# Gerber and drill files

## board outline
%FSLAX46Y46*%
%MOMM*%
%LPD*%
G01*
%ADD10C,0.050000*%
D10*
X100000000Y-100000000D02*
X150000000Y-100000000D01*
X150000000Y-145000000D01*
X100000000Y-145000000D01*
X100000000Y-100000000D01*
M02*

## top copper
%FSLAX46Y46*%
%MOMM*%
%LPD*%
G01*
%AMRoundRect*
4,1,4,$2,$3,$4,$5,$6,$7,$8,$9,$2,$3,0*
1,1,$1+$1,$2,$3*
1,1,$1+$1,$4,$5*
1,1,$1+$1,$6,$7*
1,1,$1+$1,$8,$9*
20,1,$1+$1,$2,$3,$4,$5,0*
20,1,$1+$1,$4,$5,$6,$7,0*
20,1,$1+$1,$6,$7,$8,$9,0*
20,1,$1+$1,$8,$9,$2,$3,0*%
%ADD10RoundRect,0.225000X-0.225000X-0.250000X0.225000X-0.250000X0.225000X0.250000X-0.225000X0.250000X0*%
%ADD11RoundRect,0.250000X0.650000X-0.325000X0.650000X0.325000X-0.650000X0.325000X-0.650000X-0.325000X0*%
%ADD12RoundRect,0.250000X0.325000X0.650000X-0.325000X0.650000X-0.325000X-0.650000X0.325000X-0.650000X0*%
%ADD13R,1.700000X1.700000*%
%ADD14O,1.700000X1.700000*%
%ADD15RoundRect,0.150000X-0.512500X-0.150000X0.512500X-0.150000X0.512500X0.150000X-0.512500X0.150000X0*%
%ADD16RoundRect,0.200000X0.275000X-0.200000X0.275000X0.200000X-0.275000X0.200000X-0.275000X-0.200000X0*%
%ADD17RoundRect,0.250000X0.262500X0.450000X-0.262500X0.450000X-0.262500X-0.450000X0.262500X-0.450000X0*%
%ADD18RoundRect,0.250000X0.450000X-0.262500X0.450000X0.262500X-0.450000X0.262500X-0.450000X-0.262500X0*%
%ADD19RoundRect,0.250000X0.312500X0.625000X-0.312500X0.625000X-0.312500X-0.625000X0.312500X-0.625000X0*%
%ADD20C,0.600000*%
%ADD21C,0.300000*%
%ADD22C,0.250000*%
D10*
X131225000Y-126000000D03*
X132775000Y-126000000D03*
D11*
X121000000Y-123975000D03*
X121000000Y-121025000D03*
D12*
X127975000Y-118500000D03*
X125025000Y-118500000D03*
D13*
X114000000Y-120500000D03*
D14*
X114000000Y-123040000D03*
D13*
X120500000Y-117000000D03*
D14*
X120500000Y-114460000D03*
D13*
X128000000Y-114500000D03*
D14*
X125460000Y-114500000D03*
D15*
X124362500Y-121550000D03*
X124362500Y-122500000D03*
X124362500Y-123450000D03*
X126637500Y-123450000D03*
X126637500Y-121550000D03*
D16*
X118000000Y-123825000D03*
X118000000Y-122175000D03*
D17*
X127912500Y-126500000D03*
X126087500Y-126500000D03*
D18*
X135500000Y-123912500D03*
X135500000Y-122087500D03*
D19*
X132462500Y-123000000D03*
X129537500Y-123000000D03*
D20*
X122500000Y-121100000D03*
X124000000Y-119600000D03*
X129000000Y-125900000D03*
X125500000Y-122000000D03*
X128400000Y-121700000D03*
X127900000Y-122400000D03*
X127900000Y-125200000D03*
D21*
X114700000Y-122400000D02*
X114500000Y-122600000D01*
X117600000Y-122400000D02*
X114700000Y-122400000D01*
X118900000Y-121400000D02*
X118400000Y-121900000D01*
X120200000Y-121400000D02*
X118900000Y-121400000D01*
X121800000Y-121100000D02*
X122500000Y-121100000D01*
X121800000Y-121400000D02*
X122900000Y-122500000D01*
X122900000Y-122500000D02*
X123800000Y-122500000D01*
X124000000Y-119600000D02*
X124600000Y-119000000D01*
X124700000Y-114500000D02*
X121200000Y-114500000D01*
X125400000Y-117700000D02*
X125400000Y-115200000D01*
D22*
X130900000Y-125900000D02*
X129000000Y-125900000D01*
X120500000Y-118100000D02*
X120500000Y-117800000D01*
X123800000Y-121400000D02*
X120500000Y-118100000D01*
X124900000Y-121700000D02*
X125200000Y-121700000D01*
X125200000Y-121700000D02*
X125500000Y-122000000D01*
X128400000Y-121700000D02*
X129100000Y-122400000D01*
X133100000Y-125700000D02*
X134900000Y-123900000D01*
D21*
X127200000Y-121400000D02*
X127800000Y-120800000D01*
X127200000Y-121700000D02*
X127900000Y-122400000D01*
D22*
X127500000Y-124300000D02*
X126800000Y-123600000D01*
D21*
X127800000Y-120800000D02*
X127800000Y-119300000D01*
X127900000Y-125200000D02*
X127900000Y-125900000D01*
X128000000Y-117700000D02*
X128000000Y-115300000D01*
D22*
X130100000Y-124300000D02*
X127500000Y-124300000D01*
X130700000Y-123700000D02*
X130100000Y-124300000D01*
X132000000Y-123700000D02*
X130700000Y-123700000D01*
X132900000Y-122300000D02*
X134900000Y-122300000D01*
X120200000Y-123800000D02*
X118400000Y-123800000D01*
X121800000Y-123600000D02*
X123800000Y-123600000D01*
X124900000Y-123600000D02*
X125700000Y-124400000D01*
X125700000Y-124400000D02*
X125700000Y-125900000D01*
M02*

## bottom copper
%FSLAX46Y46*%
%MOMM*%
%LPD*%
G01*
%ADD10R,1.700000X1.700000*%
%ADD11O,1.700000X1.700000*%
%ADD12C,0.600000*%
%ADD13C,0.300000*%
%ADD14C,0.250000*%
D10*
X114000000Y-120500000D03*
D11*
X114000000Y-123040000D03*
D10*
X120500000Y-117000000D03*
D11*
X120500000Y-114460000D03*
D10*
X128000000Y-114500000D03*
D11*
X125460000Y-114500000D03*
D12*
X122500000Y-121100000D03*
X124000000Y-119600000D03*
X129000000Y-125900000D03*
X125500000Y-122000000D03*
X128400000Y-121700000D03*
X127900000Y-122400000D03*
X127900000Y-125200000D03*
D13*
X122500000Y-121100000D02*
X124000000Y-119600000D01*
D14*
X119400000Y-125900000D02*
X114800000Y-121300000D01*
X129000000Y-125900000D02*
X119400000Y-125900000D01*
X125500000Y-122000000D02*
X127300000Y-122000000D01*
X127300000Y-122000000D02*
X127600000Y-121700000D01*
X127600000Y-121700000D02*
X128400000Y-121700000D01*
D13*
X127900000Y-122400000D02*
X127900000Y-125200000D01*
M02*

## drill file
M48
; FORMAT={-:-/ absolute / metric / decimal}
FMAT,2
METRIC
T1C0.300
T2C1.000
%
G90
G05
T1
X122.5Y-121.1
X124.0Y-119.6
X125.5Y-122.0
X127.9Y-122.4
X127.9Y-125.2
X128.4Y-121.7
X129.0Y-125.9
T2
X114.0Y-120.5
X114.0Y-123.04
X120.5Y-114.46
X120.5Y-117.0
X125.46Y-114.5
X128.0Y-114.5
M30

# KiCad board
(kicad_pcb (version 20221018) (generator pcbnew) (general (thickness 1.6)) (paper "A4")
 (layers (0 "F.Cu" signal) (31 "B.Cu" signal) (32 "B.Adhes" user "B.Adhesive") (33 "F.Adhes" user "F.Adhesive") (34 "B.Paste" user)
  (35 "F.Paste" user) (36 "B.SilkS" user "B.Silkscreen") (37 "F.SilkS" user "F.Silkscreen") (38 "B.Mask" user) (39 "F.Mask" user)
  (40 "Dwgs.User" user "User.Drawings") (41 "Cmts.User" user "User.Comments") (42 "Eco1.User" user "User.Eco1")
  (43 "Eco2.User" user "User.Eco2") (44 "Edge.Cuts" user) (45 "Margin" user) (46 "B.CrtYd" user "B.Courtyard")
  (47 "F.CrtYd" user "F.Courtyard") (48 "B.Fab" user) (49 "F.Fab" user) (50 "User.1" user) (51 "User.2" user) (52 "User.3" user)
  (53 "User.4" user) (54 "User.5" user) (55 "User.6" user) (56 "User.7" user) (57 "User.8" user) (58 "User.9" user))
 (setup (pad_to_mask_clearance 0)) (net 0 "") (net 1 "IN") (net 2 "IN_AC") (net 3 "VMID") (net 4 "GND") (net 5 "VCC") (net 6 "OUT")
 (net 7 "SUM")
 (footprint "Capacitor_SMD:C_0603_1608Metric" (layer "F.Cu") (at 132 126)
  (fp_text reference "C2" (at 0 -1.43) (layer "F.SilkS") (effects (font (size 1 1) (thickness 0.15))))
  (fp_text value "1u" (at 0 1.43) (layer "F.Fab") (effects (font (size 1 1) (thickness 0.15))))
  (pad "1" smd roundrect (at -0.775 0) (size 0.9 0.95) (layers "F.Cu" "F.Paste" "F.Mask") (roundrect_rratio 0.25) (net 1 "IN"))
  (pad "2" smd roundrect (at 0.775 0) (size 0.9 0.95) (layers "F.Cu" "F.Paste" "F.Mask") (roundrect_rratio 0.25) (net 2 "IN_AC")))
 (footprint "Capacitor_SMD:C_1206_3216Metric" (layer "F.Cu") (at 121 122.5 90)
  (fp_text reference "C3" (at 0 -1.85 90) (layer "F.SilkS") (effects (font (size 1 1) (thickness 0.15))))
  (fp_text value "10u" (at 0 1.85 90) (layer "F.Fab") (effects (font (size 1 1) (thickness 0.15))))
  (pad "1" smd roundrect (at -1.475 0 90) (size 1.15 1.8) (layers "F.Cu" "F.Paste" "F.Mask") (roundrect_rratio 0.217391) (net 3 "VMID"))
  (pad "2" smd roundrect (at 1.475 0 90) (size 1.15 1.8) (layers "F.Cu" "F.Paste" "F.Mask") (roundrect_rratio 0.217391) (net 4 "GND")))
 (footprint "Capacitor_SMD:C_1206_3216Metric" (layer "F.Cu") (at 126.5 118.5 180)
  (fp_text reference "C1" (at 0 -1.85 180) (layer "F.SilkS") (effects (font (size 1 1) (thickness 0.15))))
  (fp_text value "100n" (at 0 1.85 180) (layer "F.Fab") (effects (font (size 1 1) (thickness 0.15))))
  (pad "1" smd roundrect (at -1.475 0 180) (size 1.15 1.8) (layers "F.Cu" "F.Paste" "F.Mask") (roundrect_rratio 0.217391) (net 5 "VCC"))
  (pad "2" smd roundrect (at 1.475 0 180) (size 1.15 1.8) (layers "F.Cu" "F.Paste" "F.Mask") (roundrect_rratio 0.217391) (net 4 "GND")))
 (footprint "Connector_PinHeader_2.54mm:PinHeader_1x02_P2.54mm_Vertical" (layer "F.Cu") (at 114 120.5)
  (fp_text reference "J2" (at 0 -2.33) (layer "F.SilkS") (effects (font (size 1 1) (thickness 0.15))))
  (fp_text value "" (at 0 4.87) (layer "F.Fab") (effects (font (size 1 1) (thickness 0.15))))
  (pad "1" thru_hole rect (at 0 0) (size 1.7 1.7) (drill 1) (layers "*.Cu" "*.Mask") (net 1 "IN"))
  (pad "2" thru_hole oval (at 0 2.54) (size 1.7 1.7) (drill 1) (layers "*.Cu" "*.Mask") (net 4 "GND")))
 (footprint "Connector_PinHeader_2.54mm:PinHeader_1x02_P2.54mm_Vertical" (layer "F.Cu") (at 120.5 117 180)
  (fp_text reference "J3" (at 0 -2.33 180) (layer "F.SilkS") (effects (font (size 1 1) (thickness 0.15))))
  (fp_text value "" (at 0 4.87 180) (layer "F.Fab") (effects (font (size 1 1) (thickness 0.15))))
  (pad "1" thru_hole rect (at 0 0 180) (size 1.7 1.7) (drill 1) (layers "*.Cu" "*.Mask") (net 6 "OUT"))
  (pad "2" thru_hole oval (at 0 2.54 180) (size 1.7 1.7) (drill 1) (layers "*.Cu" "*.Mask") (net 4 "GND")))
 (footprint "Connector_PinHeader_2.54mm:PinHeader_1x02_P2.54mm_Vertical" (layer "F.Cu") (at 128 114.5 -90)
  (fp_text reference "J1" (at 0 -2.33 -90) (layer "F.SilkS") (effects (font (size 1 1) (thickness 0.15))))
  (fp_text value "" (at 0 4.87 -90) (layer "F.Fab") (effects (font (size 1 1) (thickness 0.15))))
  (pad "1" thru_hole rect (at 0 0 270) (size 1.7 1.7) (drill 1) (layers "*.Cu" "*.Mask") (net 5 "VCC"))
  (pad "2" thru_hole oval (at 0 2.54 270) (size 1.7 1.7) (drill 1) (layers "*.Cu" "*.Mask") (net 4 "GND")))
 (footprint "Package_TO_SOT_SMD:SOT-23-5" (layer "F.Cu") (at 125.5 122.5)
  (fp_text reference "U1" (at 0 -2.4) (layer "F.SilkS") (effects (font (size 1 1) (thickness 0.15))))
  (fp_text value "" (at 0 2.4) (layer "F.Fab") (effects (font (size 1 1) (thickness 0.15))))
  (pad "1" smd roundrect (at -1.1375 -0.95) (size 1.325 0.6) (layers "F.Cu" "F.Paste" "F.Mask") (roundrect_rratio 0.25) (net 6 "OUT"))
  (pad "2" smd roundrect (at -1.1375 0) (size 1.325 0.6) (layers "F.Cu" "F.Paste" "F.Mask") (roundrect_rratio 0.25) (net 4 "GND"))
  (pad "3" smd roundrect (at -1.1375 0.95) (size 1.325 0.6) (layers "F.Cu" "F.Paste" "F.Mask") (roundrect_rratio 0.25) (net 3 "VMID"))
  (pad "4" smd roundrect (at 1.1375 0.95) (size 1.325 0.6) (layers "F.Cu" "F.Paste" "F.Mask") (roundrect_rratio 0.25) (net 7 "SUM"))
  (pad "5" smd roundrect (at 1.1375 -0.95) (size 1.325 0.6) (layers "F.Cu" "F.Paste" "F.Mask") (roundrect_rratio 0.25) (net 5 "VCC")))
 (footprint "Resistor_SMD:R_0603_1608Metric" (layer "F.Cu") (at 118 123 90)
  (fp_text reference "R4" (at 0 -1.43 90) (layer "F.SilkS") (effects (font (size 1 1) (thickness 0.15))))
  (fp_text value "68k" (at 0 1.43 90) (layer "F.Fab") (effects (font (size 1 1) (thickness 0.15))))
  (pad "1" smd roundrect (at -0.825 0 90) (size 0.8 0.95) (layers "F.Cu" "F.Paste" "F.Mask") (roundrect_rratio 0.25) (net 3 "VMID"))
  (pad "2" smd roundrect (at 0.825 0 90) (size 0.8 0.95) (layers "F.Cu" "F.Paste" "F.Mask") (roundrect_rratio 0.25) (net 4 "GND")))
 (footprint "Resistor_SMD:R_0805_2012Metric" (layer "F.Cu") (at 127 126.5 180)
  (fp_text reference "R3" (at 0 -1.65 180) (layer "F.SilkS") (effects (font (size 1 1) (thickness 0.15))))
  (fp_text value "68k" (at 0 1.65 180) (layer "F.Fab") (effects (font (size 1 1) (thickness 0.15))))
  (pad "1" smd roundrect (at -0.9125 0 180) (size 1.025 1.4) (layers "F.Cu" "F.Paste" "F.Mask") (roundrect_rratio 0.243902) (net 5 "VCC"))
  (pad "2" smd roundrect (at 0.9125 0 180) (size 1.025 1.4) (layers "F.Cu" "F.Paste" "F.Mask") (roundrect_rratio 0.243902) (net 3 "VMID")))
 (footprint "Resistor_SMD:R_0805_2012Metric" (layer "F.Cu") (at 135.5 123 90)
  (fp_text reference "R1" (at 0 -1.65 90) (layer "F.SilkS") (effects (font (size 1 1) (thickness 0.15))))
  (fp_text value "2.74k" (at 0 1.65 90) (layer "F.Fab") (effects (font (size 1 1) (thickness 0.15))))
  (pad "1" smd roundrect (at -0.9125 0 90) (size 1.025 1.4) (layers "F.Cu" "F.Paste" "F.Mask") (roundrect_rratio 0.243902) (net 2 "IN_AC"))
  (pad "2" smd roundrect (at 0.9125 0 90) (size 1.025 1.4) (layers "F.Cu" "F.Paste" "F.Mask") (roundrect_rratio 0.243902) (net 7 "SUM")))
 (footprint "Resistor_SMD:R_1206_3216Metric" (layer "F.Cu") (at 131 123 180)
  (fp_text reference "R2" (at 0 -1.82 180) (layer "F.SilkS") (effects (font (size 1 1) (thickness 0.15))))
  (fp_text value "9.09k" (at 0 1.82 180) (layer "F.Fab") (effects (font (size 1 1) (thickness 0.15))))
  (pad "1" smd roundrect (at -1.4625 0 180) (size 1.125 1.75) (layers "F.Cu" "F.Paste" "F.Mask") (roundrect_rratio 0.222222) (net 7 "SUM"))
  (pad "2" smd roundrect (at 1.4625 0 180) (size 1.125 1.75) (layers "F.Cu" "F.Paste" "F.Mask") (roundrect_rratio 0.222222) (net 6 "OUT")))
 (gr_rect (start 100 100) (end 150 145) (stroke (width 0.05) (type default)) (fill none) (layer "Edge.Cuts"))
 (segment (start 114.7 122.4) (end 114.5 122.6) (width 0.3) (layer "F.Cu") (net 4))
 (segment (start 117.6 122.4) (end 114.7 122.4) (width 0.3) (layer "F.Cu") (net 4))
 (segment (start 118.9 121.4) (end 118.4 121.9) (width 0.3) (layer "F.Cu") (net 4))
 (segment (start 120.2 121.4) (end 118.9 121.4) (width 0.3) (layer "F.Cu") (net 4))
 (segment (start 121.8 121.1) (end 122.5 121.1) (width 0.3) (layer "F.Cu") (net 4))
 (segment (start 121.8 121.4) (end 122.9 122.5) (width 0.3) (layer "F.Cu") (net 4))
 (segment (start 122.9 122.5) (end 123.8 122.5) (width 0.3) (layer "F.Cu") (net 4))
 (segment (start 124 119.6) (end 124.6 119) (width 0.3) (layer "F.Cu") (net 4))
 (segment (start 124.7 114.5) (end 121.2 114.5) (width 0.3) (layer "F.Cu") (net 4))
 (segment (start 125.4 117.7) (end 125.4 115.2) (width 0.3) (layer "F.Cu") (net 4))
 (via (at 122.5 121.1) (size 0.6) (drill 0.3) (layers "F.Cu" "B.Cu") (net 4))
 (via (at 124 119.6) (size 0.6) (drill 0.3) (layers "F.Cu" "B.Cu") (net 4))
 (segment (start 122.5 121.1) (end 124 119.6) (width 0.3) (layer "B.Cu") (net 4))
 (segment (start 130.9 125.9) (end 129 125.9) (width 0.25) (layer "F.Cu") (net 1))
 (via (at 129 125.9) (size 0.6) (drill 0.3) (layers "F.Cu" "B.Cu") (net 1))
 (segment (start 119.4 125.9) (end 114.8 121.3) (width 0.25) (layer "B.Cu") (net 1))
 (segment (start 120.5 118.1) (end 120.5 117.8) (width 0.25) (layer "F.Cu") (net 6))
 (segment (start 123.8 121.4) (end 120.5 118.1) (width 0.25) (layer "F.Cu") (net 6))
 (segment (start 124.9 121.7) (end 125.2 121.7) (width 0.25) (layer "F.Cu") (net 6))
 (segment (start 125.2 121.7) (end 125.5 122) (width 0.25) (layer "F.Cu") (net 6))
 (segment (start 128.4 121.7) (end 129.1 122.4) (width 0.25) (layer "F.Cu") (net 6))
 (segment (start 129 125.9) (end 119.4 125.9) (width 0.25) (layer "B.Cu") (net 1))
 (segment (start 133.1 125.7) (end 134.9 123.9) (width 0.25) (layer "F.Cu") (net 2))
 (via (at 125.5 122) (size 0.6) (drill 0.3) (layers "F.Cu" "B.Cu") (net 6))
 (via (at 128.4 121.7) (size 0.6) (drill 0.3) (layers "F.Cu" "B.Cu") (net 6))
 (segment (start 125.5 122) (end 127.3 122) (width 0.25) (layer "B.Cu") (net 6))
 (segment (start 127.2 121.4) (end 127.8 120.8) (width 0.3) (layer "F.Cu") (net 5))
 (segment (start 127.2 121.7) (end 127.9 122.4) (width 0.3) (layer "F.Cu") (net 5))
 (segment (start 127.3 122) (end 127.6 121.7) (width 0.25) (layer "B.Cu") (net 6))
 (segment (start 127.5 124.3) (end 126.8 123.6) (width 0.25) (layer "F.Cu") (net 7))
 (segment (start 127.6 121.7) (end 128.4 121.7) (width 0.25) (layer "B.Cu") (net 6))
 (segment (start 127.8 120.8) (end 127.8 119.3) (width 0.3) (layer "F.Cu") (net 5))
 (segment (start 127.9 125.2) (end 127.9 125.9) (width 0.3) (layer "F.Cu") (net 5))
 (segment (start 128 117.7) (end 128 115.3) (width 0.3) (layer "F.Cu") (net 5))
 (segment (start 130.1 124.3) (end 127.5 124.3) (width 0.25) (layer "F.Cu") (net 7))
 (segment (start 130.7 123.7) (end 130.1 124.3) (width 0.25) (layer "F.Cu") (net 7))
 (segment (start 132 123.7) (end 130.7 123.7) (width 0.25) (layer "F.Cu") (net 7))
 (segment (start 132.9 122.3) (end 134.9 122.3) (width 0.25) (layer "F.Cu") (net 7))
 (via (at 127.9 122.4) (size 0.6) (drill 0.3) (layers "F.Cu" "B.Cu") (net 5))
 (via (at 127.9 125.2) (size 0.6) (drill 0.3) (layers "F.Cu" "B.Cu") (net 5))
 (segment (start 120.2 123.8) (end 118.4 123.8) (width 0.25) (layer "F.Cu") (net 3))
 (segment (start 121.8 123.6) (end 123.8 123.6) (width 0.25) (layer "F.Cu") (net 3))
 (segment (start 124.9 123.6) (end 125.7 124.4) (width 0.25) (layer "F.Cu") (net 3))
 (segment (start 125.7 124.4) (end 125.7 125.9) (width 0.25) (layer "F.Cu") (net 3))
 (segment (start 127.9 122.4) (end 127.9 125.2) (width 0.3) (layer "B.Cu") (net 5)))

